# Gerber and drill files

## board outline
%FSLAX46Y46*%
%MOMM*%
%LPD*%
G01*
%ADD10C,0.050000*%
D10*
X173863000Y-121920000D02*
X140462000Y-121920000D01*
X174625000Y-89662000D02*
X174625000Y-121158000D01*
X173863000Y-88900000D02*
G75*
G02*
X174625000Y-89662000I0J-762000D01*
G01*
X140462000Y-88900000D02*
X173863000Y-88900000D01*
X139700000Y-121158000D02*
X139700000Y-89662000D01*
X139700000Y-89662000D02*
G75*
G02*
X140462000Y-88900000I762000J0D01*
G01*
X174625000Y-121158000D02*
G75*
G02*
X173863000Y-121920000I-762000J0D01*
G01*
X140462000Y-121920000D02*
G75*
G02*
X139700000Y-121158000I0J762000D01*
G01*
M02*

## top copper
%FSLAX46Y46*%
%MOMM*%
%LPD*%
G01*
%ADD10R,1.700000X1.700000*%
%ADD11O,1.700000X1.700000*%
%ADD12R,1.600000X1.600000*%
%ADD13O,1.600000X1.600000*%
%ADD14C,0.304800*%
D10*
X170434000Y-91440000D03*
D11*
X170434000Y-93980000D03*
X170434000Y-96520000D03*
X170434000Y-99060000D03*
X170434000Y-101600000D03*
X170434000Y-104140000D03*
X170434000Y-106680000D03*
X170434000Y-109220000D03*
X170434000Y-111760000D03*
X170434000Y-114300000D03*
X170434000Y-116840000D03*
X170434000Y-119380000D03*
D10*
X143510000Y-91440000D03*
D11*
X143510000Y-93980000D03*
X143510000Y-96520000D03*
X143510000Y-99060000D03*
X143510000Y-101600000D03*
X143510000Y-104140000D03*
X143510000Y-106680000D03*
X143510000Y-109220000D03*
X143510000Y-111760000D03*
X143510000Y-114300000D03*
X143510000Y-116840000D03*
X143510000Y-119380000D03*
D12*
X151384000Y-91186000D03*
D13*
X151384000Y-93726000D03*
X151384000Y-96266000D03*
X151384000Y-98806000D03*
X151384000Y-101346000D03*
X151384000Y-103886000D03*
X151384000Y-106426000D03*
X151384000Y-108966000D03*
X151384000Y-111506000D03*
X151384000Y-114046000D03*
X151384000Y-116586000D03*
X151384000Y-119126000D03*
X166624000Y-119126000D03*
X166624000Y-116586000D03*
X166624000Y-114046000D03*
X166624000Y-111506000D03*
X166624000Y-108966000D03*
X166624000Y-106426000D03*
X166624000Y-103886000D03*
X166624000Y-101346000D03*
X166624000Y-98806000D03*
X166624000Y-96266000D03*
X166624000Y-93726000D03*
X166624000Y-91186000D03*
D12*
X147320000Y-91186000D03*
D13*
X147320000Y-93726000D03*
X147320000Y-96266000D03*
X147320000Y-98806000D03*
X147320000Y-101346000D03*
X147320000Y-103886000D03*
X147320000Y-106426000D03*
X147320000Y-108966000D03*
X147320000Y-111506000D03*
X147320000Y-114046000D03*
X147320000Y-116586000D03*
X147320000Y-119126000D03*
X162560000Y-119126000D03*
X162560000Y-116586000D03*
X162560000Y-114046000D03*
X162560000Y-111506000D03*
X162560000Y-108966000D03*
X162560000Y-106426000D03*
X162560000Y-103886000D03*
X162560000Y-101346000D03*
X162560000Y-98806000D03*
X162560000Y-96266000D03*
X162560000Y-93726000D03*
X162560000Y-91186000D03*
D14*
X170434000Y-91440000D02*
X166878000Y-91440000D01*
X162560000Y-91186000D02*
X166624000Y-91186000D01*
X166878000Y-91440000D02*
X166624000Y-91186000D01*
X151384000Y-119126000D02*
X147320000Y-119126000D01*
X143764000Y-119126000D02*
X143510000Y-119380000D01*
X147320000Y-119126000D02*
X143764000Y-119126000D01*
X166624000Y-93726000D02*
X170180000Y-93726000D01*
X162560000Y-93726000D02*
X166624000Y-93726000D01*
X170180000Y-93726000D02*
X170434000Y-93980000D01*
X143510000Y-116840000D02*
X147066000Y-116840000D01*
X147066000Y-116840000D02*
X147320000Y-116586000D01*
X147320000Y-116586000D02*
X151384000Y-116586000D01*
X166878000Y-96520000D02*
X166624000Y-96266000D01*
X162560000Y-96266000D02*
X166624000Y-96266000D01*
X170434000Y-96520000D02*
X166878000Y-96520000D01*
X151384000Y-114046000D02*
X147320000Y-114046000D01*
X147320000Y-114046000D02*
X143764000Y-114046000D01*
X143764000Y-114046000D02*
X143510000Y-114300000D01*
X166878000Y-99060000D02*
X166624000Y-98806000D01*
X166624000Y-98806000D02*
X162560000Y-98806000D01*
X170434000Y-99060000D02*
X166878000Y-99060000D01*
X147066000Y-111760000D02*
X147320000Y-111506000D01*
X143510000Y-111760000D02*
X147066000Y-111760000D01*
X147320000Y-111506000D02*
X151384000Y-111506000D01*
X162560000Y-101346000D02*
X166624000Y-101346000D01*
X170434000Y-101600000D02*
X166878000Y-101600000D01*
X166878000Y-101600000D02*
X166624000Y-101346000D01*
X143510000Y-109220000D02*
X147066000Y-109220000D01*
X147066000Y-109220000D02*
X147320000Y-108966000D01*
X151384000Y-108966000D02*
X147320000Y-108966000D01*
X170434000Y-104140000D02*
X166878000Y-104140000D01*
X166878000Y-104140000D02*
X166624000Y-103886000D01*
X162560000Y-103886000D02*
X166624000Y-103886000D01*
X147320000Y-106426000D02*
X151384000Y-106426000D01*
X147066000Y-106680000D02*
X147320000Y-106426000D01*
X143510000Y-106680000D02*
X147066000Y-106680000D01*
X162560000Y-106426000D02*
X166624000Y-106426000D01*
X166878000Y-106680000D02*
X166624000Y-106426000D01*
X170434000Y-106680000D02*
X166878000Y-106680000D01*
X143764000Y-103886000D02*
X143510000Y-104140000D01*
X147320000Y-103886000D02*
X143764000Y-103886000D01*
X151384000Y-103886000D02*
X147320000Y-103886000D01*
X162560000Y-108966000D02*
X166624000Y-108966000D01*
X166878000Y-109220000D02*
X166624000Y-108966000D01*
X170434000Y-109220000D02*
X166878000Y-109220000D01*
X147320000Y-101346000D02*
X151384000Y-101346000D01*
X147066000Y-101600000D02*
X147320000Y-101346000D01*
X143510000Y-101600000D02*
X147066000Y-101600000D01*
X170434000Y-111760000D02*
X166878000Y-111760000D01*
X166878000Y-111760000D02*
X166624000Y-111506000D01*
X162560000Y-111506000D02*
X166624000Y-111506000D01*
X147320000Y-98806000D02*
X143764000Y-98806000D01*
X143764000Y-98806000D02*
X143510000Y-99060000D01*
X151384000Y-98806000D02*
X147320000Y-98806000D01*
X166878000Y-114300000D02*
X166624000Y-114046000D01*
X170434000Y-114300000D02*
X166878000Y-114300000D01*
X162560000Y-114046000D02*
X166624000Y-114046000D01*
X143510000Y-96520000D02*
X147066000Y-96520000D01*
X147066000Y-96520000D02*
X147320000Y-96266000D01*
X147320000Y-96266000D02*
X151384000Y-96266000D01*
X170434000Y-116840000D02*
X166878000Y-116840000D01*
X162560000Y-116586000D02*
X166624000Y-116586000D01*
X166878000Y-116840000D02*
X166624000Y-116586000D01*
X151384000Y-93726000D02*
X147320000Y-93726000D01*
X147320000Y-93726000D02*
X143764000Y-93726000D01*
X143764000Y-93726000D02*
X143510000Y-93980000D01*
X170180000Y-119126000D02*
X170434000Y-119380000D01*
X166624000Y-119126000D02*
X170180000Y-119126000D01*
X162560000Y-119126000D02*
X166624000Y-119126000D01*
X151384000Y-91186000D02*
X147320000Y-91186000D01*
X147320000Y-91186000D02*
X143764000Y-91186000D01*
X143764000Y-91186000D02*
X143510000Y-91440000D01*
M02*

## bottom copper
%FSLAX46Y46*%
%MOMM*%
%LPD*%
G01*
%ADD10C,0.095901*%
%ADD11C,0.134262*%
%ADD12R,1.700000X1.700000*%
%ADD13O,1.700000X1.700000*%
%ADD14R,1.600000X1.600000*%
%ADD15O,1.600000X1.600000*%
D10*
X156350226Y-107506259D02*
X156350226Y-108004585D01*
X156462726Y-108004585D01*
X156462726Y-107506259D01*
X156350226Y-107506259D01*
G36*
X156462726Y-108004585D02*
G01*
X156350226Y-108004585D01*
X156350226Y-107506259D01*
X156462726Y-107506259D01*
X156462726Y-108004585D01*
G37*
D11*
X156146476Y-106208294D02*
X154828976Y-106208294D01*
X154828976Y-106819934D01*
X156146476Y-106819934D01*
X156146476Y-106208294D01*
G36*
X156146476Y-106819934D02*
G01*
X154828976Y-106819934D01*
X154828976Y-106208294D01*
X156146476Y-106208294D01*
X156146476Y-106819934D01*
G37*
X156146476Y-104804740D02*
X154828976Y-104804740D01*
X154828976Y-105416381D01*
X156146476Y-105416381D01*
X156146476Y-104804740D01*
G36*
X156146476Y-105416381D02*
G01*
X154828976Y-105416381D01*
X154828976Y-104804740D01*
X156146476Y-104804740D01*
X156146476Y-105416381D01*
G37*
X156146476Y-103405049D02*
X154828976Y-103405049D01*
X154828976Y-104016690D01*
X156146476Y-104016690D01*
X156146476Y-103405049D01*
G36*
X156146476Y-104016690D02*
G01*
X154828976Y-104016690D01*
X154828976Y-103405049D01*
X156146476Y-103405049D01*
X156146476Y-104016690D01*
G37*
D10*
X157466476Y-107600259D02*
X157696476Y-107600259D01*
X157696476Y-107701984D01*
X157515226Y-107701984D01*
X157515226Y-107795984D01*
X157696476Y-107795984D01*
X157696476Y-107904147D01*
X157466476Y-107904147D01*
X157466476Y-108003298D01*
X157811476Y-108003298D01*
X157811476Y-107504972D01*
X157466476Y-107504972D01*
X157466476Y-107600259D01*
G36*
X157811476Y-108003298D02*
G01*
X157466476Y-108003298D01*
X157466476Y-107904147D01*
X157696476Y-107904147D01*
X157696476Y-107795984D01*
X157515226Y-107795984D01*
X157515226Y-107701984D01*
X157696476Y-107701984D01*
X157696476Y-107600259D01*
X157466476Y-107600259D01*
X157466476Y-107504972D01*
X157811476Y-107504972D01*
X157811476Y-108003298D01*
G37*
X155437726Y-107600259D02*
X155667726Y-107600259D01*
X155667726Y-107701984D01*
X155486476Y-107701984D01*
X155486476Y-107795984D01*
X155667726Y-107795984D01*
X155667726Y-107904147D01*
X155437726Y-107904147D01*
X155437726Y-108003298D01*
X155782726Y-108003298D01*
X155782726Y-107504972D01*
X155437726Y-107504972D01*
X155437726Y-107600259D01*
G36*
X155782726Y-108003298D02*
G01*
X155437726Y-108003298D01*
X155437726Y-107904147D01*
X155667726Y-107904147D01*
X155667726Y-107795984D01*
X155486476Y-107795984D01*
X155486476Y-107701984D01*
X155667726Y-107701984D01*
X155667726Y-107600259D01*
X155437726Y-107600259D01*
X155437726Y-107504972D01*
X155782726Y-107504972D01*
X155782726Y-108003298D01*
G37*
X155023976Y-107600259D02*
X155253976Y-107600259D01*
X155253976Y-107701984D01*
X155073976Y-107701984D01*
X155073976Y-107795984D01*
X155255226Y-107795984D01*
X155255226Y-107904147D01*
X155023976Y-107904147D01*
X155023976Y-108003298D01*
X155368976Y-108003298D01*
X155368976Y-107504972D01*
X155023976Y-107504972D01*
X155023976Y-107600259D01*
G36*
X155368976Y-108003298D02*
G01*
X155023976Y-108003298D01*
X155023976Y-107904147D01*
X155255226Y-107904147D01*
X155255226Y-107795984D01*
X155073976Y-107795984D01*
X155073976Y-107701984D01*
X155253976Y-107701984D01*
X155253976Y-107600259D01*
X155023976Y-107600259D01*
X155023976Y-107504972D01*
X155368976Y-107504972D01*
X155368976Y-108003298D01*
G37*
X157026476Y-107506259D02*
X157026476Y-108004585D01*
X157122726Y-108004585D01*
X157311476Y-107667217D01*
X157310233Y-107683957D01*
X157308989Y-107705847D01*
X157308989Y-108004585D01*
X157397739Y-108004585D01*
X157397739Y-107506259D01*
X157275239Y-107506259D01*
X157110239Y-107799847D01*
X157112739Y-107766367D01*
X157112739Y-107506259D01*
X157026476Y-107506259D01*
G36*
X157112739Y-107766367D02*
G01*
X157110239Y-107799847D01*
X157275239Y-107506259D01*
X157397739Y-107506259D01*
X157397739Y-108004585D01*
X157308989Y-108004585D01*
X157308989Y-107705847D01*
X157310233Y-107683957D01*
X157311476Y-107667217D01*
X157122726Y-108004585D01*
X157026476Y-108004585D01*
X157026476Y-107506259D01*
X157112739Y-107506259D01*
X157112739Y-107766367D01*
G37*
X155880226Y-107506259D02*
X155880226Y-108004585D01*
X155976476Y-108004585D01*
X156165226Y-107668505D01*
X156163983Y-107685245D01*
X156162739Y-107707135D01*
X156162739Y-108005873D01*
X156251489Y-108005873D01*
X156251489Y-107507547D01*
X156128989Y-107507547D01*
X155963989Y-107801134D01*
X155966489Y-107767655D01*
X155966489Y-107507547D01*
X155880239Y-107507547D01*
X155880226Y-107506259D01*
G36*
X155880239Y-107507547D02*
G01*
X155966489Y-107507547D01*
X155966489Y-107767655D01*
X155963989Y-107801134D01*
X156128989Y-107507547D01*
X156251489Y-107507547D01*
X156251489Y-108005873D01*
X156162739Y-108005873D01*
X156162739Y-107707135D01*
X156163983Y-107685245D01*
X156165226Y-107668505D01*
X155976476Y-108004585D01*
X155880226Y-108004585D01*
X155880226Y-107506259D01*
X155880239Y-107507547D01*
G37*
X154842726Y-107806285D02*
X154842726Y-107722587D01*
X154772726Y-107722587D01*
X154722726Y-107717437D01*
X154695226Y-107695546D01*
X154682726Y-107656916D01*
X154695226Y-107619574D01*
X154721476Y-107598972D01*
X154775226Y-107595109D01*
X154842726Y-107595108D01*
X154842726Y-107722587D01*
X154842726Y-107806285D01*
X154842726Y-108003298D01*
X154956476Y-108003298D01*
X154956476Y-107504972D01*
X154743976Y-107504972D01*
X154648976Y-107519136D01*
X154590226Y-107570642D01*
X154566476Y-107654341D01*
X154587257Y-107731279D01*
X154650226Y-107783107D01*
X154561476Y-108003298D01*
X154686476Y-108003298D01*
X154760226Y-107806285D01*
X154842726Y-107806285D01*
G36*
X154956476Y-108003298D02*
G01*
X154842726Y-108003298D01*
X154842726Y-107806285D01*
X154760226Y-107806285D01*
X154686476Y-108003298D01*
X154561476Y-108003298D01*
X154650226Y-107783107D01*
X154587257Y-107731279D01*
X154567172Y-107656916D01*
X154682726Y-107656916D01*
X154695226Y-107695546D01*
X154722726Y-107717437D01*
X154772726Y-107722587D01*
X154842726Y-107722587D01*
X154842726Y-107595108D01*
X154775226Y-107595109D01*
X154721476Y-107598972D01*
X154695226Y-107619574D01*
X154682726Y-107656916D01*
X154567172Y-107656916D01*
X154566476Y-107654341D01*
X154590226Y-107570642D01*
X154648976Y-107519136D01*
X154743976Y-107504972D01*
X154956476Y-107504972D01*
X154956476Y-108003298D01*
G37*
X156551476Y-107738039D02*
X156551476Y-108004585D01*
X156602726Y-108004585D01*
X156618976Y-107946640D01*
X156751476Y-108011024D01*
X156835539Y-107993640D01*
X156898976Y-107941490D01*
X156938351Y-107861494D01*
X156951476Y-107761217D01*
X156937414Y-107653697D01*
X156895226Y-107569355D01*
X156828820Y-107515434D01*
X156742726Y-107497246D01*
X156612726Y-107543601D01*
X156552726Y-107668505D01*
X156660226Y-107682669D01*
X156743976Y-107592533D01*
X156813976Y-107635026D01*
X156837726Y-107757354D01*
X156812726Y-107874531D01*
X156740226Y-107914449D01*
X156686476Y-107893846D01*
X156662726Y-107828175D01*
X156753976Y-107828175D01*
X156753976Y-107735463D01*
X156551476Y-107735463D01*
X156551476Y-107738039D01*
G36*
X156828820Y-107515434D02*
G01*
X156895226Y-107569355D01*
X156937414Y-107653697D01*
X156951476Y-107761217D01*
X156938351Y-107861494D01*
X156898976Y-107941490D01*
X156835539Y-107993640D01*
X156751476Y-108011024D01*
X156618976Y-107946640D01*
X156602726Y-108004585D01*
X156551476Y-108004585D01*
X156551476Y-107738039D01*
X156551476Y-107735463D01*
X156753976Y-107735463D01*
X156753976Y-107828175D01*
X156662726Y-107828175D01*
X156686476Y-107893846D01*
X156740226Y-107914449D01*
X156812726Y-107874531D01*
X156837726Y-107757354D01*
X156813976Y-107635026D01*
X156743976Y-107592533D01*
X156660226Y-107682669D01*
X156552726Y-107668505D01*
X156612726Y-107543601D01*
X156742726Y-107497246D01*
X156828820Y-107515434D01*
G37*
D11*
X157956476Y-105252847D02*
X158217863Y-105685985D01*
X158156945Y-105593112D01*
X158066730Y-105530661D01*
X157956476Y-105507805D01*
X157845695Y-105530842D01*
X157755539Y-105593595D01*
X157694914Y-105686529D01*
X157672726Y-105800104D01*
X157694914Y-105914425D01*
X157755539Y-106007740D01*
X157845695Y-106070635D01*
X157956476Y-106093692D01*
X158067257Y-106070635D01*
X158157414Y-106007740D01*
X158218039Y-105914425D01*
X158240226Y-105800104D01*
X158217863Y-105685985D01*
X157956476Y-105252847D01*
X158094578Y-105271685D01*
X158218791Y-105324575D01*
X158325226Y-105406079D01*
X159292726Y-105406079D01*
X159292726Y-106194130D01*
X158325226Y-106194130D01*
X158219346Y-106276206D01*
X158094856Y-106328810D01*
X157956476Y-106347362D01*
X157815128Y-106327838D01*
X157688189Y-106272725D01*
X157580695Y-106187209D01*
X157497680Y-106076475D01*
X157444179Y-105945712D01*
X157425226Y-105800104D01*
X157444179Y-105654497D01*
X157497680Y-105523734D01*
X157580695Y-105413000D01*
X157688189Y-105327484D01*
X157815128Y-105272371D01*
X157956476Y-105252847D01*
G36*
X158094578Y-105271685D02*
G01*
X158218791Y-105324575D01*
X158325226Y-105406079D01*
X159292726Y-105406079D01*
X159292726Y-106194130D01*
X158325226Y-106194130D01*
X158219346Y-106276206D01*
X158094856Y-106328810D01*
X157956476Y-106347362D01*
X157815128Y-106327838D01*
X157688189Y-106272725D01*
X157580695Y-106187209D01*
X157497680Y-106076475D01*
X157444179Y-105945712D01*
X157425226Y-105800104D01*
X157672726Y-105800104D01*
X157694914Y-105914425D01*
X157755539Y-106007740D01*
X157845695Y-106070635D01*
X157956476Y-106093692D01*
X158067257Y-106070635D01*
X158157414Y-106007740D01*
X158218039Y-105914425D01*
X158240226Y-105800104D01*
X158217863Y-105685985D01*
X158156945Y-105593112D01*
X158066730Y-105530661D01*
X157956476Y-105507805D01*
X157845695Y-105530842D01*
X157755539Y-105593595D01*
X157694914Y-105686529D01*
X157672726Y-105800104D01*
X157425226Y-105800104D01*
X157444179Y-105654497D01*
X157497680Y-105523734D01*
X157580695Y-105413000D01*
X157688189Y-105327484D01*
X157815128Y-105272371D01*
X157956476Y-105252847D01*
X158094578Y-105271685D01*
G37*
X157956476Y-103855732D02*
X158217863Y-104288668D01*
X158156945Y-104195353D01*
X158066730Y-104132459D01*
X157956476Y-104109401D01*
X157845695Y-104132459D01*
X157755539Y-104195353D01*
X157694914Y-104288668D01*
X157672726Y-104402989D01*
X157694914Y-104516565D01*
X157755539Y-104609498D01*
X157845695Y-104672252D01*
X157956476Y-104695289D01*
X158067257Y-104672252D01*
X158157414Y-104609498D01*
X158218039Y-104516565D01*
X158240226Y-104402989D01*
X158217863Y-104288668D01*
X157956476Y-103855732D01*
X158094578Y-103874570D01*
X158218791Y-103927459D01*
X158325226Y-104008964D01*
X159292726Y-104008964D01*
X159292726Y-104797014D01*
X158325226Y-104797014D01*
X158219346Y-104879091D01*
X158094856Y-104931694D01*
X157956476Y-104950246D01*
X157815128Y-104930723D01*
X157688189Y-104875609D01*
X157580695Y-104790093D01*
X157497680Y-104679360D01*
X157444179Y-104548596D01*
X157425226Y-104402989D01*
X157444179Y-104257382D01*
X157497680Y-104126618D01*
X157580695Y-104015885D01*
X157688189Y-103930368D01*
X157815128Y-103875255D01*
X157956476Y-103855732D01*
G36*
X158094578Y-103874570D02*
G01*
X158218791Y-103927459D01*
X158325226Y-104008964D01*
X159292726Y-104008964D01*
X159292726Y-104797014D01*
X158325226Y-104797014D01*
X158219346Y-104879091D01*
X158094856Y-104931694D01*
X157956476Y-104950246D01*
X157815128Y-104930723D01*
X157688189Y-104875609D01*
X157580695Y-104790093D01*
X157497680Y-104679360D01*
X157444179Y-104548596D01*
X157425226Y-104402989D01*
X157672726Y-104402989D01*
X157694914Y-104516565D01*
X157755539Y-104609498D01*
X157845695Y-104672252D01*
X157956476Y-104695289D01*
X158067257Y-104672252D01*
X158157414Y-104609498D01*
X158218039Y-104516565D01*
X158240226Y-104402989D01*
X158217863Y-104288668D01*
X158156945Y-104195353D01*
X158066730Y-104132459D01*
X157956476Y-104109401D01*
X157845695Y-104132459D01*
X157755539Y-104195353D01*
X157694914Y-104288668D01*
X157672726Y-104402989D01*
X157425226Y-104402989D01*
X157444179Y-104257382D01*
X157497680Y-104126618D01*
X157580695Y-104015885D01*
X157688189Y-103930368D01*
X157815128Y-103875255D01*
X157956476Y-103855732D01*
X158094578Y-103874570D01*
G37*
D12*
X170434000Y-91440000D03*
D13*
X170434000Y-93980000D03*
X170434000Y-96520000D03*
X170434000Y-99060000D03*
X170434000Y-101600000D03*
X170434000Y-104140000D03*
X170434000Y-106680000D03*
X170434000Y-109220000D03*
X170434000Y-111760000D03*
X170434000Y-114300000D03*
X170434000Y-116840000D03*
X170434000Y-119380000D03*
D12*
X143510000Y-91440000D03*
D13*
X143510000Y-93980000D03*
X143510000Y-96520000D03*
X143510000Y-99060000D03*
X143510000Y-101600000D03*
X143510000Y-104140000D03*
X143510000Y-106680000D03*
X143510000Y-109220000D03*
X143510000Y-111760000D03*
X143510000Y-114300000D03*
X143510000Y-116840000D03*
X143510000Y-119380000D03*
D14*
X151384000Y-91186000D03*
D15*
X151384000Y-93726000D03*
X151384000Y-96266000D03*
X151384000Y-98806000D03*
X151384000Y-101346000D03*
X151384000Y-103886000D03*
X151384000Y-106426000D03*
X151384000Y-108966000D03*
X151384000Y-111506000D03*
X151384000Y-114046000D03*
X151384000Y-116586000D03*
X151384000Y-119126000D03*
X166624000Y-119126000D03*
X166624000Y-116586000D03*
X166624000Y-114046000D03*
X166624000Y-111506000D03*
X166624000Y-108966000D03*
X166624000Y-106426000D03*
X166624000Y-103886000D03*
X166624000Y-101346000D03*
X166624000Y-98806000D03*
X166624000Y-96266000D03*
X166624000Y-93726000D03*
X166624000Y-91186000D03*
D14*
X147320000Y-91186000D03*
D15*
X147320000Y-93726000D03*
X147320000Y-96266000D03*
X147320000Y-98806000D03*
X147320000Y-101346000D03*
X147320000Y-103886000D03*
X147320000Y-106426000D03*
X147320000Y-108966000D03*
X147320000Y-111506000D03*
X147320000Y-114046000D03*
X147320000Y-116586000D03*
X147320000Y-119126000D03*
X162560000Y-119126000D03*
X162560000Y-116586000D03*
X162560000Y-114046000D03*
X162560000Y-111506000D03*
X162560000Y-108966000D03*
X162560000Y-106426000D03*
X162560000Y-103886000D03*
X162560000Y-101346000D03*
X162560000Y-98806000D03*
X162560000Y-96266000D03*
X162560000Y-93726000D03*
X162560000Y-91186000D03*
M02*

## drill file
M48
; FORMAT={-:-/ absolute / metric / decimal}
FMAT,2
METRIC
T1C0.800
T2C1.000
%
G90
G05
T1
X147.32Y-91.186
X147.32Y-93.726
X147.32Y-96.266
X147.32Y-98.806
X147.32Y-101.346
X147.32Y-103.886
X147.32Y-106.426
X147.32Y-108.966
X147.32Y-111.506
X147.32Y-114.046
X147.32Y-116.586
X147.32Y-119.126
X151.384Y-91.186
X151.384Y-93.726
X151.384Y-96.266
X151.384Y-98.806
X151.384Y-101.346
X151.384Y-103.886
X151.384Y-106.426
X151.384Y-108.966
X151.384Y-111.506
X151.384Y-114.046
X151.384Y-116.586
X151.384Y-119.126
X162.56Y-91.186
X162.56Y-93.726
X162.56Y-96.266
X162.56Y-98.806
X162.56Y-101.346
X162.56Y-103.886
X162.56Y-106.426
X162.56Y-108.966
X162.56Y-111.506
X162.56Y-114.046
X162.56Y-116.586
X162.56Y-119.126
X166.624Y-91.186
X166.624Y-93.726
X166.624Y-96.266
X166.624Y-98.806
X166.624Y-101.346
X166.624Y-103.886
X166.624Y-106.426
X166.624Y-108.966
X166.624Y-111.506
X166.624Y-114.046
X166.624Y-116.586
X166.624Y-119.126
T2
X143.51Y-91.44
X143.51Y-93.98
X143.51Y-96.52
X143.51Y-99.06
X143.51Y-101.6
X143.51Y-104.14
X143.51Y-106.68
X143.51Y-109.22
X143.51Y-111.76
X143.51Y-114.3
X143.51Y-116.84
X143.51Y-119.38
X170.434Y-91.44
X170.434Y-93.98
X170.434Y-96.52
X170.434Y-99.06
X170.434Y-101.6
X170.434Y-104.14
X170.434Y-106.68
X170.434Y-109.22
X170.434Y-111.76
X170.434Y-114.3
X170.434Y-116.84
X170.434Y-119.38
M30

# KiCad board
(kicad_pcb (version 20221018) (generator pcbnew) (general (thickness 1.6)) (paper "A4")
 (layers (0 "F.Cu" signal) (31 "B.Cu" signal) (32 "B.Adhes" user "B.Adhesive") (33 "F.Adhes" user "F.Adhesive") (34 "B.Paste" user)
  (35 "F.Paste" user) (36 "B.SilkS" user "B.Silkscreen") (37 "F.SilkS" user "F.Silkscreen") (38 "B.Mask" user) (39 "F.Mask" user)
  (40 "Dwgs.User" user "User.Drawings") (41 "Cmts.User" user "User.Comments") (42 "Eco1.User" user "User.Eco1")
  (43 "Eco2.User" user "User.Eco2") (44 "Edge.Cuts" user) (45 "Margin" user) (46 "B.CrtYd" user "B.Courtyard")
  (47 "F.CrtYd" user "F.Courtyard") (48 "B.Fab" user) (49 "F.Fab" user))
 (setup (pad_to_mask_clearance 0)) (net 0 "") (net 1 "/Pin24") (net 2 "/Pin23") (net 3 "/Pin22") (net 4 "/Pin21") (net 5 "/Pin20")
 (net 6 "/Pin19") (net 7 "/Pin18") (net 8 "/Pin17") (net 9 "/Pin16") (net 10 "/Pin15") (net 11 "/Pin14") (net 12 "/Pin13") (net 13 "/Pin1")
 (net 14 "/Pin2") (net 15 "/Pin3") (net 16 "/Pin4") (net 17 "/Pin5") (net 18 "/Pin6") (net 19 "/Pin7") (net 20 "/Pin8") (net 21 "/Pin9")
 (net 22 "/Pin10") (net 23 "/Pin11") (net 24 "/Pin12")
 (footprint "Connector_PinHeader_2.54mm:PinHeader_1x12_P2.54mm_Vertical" (layer "F.Cu") (at 170.434 91.44)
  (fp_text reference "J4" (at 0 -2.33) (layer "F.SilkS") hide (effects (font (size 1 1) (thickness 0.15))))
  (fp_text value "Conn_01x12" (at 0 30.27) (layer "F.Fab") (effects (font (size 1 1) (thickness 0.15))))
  (pad "1" thru_hole rect (at 0 0) (size 1.7 1.7) (drill 1) (layers "*.Cu" "*.Mask") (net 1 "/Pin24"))
  (pad "2" thru_hole oval (at 0 2.54) (size 1.7 1.7) (drill 1) (layers "*.Cu" "*.Mask") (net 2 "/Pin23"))
  (pad "3" thru_hole oval (at 0 5.08) (size 1.7 1.7) (drill 1) (layers "*.Cu" "*.Mask") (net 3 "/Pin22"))
  (pad "4" thru_hole oval (at 0 7.62) (size 1.7 1.7) (drill 1) (layers "*.Cu" "*.Mask") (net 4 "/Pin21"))
  (pad "5" thru_hole oval (at 0 10.16) (size 1.7 1.7) (drill 1) (layers "*.Cu" "*.Mask") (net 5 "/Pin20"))
  (pad "6" thru_hole oval (at 0 12.7) (size 1.7 1.7) (drill 1) (layers "*.Cu" "*.Mask") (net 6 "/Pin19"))
  (pad "7" thru_hole oval (at 0 15.24) (size 1.7 1.7) (drill 1) (layers "*.Cu" "*.Mask") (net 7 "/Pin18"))
  (pad "8" thru_hole oval (at 0 17.78) (size 1.7 1.7) (drill 1) (layers "*.Cu" "*.Mask") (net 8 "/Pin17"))
  (pad "9" thru_hole oval (at 0 20.32) (size 1.7 1.7) (drill 1) (layers "*.Cu" "*.Mask") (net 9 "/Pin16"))
  (pad "10" thru_hole oval (at 0 22.86) (size 1.7 1.7) (drill 1) (layers "*.Cu" "*.Mask") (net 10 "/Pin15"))
  (pad "11" thru_hole oval (at 0 25.4) (size 1.7 1.7) (drill 1) (layers "*.Cu" "*.Mask") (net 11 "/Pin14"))
  (pad "12" thru_hole oval (at 0 27.94) (size 1.7 1.7) (drill 1) (layers "*.Cu" "*.Mask") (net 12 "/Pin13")))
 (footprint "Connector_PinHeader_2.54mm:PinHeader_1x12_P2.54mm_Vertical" (layer "F.Cu") (at 143.51 91.44)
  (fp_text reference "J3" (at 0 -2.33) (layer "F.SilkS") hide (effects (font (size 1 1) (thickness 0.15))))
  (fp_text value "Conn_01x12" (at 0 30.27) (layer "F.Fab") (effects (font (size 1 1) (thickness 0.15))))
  (pad "1" thru_hole rect (at 0 0) (size 1.7 1.7) (drill 1) (layers "*.Cu" "*.Mask") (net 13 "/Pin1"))
  (pad "2" thru_hole oval (at 0 2.54) (size 1.7 1.7) (drill 1) (layers "*.Cu" "*.Mask") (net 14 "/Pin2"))
  (pad "3" thru_hole oval (at 0 5.08) (size 1.7 1.7) (drill 1) (layers "*.Cu" "*.Mask") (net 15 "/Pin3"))
  (pad "4" thru_hole oval (at 0 7.62) (size 1.7 1.7) (drill 1) (layers "*.Cu" "*.Mask") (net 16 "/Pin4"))
  (pad "5" thru_hole oval (at 0 10.16) (size 1.7 1.7) (drill 1) (layers "*.Cu" "*.Mask") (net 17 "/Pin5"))
  (pad "6" thru_hole oval (at 0 12.7) (size 1.7 1.7) (drill 1) (layers "*.Cu" "*.Mask") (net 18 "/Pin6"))
  (pad "7" thru_hole oval (at 0 15.24) (size 1.7 1.7) (drill 1) (layers "*.Cu" "*.Mask") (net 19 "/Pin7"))
  (pad "8" thru_hole oval (at 0 17.78) (size 1.7 1.7) (drill 1) (layers "*.Cu" "*.Mask") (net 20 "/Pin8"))
  (pad "9" thru_hole oval (at 0 20.32) (size 1.7 1.7) (drill 1) (layers "*.Cu" "*.Mask") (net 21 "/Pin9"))
  (pad "10" thru_hole oval (at 0 22.86) (size 1.7 1.7) (drill 1) (layers "*.Cu" "*.Mask") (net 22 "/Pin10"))
  (pad "11" thru_hole oval (at 0 25.4) (size 1.7 1.7) (drill 1) (layers "*.Cu" "*.Mask") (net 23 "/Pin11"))
  (pad "12" thru_hole oval (at 0 27.94) (size 1.7 1.7) (drill 1) (layers "*.Cu" "*.Mask") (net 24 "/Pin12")))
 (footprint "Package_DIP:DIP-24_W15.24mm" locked (layer "F.Cu") (at 151.384 91.186)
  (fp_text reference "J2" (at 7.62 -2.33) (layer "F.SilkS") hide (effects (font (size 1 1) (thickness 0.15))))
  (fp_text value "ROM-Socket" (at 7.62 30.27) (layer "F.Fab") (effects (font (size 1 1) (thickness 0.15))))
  (pad "1" thru_hole rect locked (at 0 0) (size 1.6 1.6) (drill 0.8) (layers "*.Cu" "*.Mask") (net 13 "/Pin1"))
  (pad "2" thru_hole oval locked (at 0 2.54) (size 1.6 1.6) (drill 0.8) (layers "*.Cu" "*.Mask") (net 14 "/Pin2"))
  (pad "3" thru_hole oval locked (at 0 5.08) (size 1.6 1.6) (drill 0.8) (layers "*.Cu" "*.Mask") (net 15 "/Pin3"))
  (pad "4" thru_hole oval locked (at 0 7.62) (size 1.6 1.6) (drill 0.8) (layers "*.Cu" "*.Mask") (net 16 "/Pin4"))
  (pad "5" thru_hole oval locked (at 0 10.16) (size 1.6 1.6) (drill 0.8) (layers "*.Cu" "*.Mask") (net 17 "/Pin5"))
  (pad "6" thru_hole oval locked (at 0 12.7) (size 1.6 1.6) (drill 0.8) (layers "*.Cu" "*.Mask") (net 18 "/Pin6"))
  (pad "7" thru_hole oval locked (at 0 15.24) (size 1.6 1.6) (drill 0.8) (layers "*.Cu" "*.Mask") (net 19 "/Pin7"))
  (pad "8" thru_hole oval locked (at 0 17.78) (size 1.6 1.6) (drill 0.8) (layers "*.Cu" "*.Mask") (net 20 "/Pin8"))
  (pad "9" thru_hole oval locked (at 0 20.32) (size 1.6 1.6) (drill 0.8) (layers "*.Cu" "*.Mask") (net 21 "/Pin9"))
  (pad "10" thru_hole oval locked (at 0 22.86) (size 1.6 1.6) (drill 0.8) (layers "*.Cu" "*.Mask") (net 22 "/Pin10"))
  (pad "11" thru_hole oval locked (at 0 25.4) (size 1.6 1.6) (drill 0.8) (layers "*.Cu" "*.Mask") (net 23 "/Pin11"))
  (pad "12" thru_hole oval locked (at 0 27.94) (size 1.6 1.6) (drill 0.8) (layers "*.Cu" "*.Mask") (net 24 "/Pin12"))
  (pad "13" thru_hole oval locked (at 15.24 27.94) (size 1.6 1.6) (drill 0.8) (layers "*.Cu" "*.Mask") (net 12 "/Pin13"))
  (pad "14" thru_hole oval locked (at 15.24 25.4) (size 1.6 1.6) (drill 0.8) (layers "*.Cu" "*.Mask") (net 11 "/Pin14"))
  (pad "15" thru_hole oval locked (at 15.24 22.86) (size 1.6 1.6) (drill 0.8) (layers "*.Cu" "*.Mask") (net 10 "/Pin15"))
  (pad "16" thru_hole oval locked (at 15.24 20.32) (size 1.6 1.6) (drill 0.8) (layers "*.Cu" "*.Mask") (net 9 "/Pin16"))
  (pad "17" thru_hole oval locked (at 15.24 17.78) (size 1.6 1.6) (drill 0.8) (layers "*.Cu" "*.Mask") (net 8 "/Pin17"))
  (pad "18" thru_hole oval locked (at 15.24 15.24) (size 1.6 1.6) (drill 0.8) (layers "*.Cu" "*.Mask") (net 7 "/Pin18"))
  (pad "19" thru_hole oval locked (at 15.24 12.7) (size 1.6 1.6) (drill 0.8) (layers "*.Cu" "*.Mask") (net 6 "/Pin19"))
  (pad "20" thru_hole oval locked (at 15.24 10.16) (size 1.6 1.6) (drill 0.8) (layers "*.Cu" "*.Mask") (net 5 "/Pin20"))
  (pad "21" thru_hole oval locked (at 15.24 7.62) (size 1.6 1.6) (drill 0.8) (layers "*.Cu" "*.Mask") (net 4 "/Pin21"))
  (pad "22" thru_hole oval locked (at 15.24 5.08) (size 1.6 1.6) (drill 0.8) (layers "*.Cu" "*.Mask") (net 3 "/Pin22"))
  (pad "23" thru_hole oval locked (at 15.24 2.54) (size 1.6 1.6) (drill 0.8) (layers "*.Cu" "*.Mask") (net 2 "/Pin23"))
  (pad "24" thru_hole oval locked (at 15.24 0) (size 1.6 1.6) (drill 0.8) (layers "*.Cu" "*.Mask") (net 1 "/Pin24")))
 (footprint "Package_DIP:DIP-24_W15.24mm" (layer "F.Cu") (at 147.32 91.186)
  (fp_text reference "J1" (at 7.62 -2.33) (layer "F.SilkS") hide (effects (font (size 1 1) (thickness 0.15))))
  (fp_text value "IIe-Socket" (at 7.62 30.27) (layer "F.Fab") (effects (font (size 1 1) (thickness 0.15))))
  (pad "1" thru_hole rect (at 0 0) (size 1.6 1.6) (drill 0.8) (layers "*.Cu" "*.Mask") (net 13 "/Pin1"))
  (pad "2" thru_hole oval (at 0 2.54) (size 1.6 1.6) (drill 0.8) (layers "*.Cu" "*.Mask") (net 14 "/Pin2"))
  (pad "3" thru_hole oval (at 0 5.08) (size 1.6 1.6) (drill 0.8) (layers "*.Cu" "*.Mask") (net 15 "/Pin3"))
  (pad "4" thru_hole oval (at 0 7.62) (size 1.6 1.6) (drill 0.8) (layers "*.Cu" "*.Mask") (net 16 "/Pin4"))
  (pad "5" thru_hole oval (at 0 10.16) (size 1.6 1.6) (drill 0.8) (layers "*.Cu" "*.Mask") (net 17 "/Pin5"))
  (pad "6" thru_hole oval (at 0 12.7) (size 1.6 1.6) (drill 0.8) (layers "*.Cu" "*.Mask") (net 18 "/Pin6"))
  (pad "7" thru_hole oval (at 0 15.24) (size 1.6 1.6) (drill 0.8) (layers "*.Cu" "*.Mask") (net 19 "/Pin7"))
  (pad "8" thru_hole oval (at 0 17.78) (size 1.6 1.6) (drill 0.8) (layers "*.Cu" "*.Mask") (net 20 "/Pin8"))
  (pad "9" thru_hole oval (at 0 20.32) (size 1.6 1.6) (drill 0.8) (layers "*.Cu" "*.Mask") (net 21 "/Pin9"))
  (pad "10" thru_hole oval (at 0 22.86) (size 1.6 1.6) (drill 0.8) (layers "*.Cu" "*.Mask") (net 22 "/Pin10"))
  (pad "11" thru_hole oval (at 0 25.4) (size 1.6 1.6) (drill 0.8) (layers "*.Cu" "*.Mask") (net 23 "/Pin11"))
  (pad "12" thru_hole oval (at 0 27.94) (size 1.6 1.6) (drill 0.8) (layers "*.Cu" "*.Mask") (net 24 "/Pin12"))
  (pad "13" thru_hole oval (at 15.24 27.94) (size 1.6 1.6) (drill 0.8) (layers "*.Cu" "*.Mask") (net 12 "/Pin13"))
  (pad "14" thru_hole oval (at 15.24 25.4) (size 1.6 1.6) (drill 0.8) (layers "*.Cu" "*.Mask") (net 11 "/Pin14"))
  (pad "15" thru_hole oval (at 15.24 22.86) (size 1.6 1.6) (drill 0.8) (layers "*.Cu" "*.Mask") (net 10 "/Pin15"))
  (pad "16" thru_hole oval (at 15.24 20.32) (size 1.6 1.6) (drill 0.8) (layers "*.Cu" "*.Mask") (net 9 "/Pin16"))
  (pad "17" thru_hole oval (at 15.24 17.78) (size 1.6 1.6) (drill 0.8) (layers "*.Cu" "*.Mask") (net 8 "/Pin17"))
  (pad "18" thru_hole oval (at 15.24 15.24) (size 1.6 1.6) (drill 0.8) (layers "*.Cu" "*.Mask") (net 7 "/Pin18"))
  (pad "19" thru_hole oval (at 15.24 12.7) (size 1.6 1.6) (drill 0.8) (layers "*.Cu" "*.Mask") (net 6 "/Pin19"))
  (pad "20" thru_hole oval (at 15.24 10.16) (size 1.6 1.6) (drill 0.8) (layers "*.Cu" "*.Mask") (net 5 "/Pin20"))
  (pad "21" thru_hole oval (at 15.24 7.62) (size 1.6 1.6) (drill 0.8) (layers "*.Cu" "*.Mask") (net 4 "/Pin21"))
  (pad "22" thru_hole oval (at 15.24 5.08) (size 1.6 1.6) (drill 0.8) (layers "*.Cu" "*.Mask") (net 3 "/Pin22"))
  (pad "23" thru_hole oval (at 15.24 2.54) (size 1.6 1.6) (drill 0.8) (layers "*.Cu" "*.Mask") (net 2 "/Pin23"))
  (pad "24" thru_hole oval (at 15.24 0) (size 1.6 1.6) (drill 0.8) (layers "*.Cu" "*.Mask") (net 1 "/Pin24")))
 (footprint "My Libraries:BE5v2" (layer "B.Cu") (at 159.561476 103.011024 180)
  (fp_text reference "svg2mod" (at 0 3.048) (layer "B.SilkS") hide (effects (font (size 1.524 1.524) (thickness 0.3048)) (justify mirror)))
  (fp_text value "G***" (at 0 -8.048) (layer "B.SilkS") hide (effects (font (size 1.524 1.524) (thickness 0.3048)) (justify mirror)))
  (fp_poly
   (pts (xy 3.21125 -4.495235) (xy 3.21125 -4.993561) (xy 3.09875 -4.993561) (xy 3.09875 -4.495235) (xy 3.21125 -4.495235))
   (stroke (width 0.095901) (type solid)) (fill solid) (layer "B.Cu"))
  (fp_poly
   (pts (xy 3.415 -3.19727) (xy 4.7325 -3.19727) (xy 4.7325 -3.80891) (xy 3.415 -3.80891) (xy 3.415 -3.19727))
   (stroke (width 0.134262) (type solid)) (fill solid) (layer "B.Cu"))
  (fp_poly
   (pts (xy 3.415 -1.793716) (xy 4.7325 -1.793716) (xy 4.7325 -2.405357) (xy 3.415 -2.405357) (xy 3.415 -1.793716))
   (stroke (width 0.134262) (type solid)) (fill solid) (layer "B.Cu"))
  (fp_poly
   (pts (xy 3.415 -0.394025) (xy 4.7325 -0.394025) (xy 4.7325 -1.005666) (xy 3.415 -1.005666) (xy 3.415 -0.394025))
   (stroke (width 0.134262) (type solid)) (fill solid) (layer "B.Cu"))
  (fp_poly
   (pts (xy 2.095 -4.589235) (xy 1.865 -4.589235) (xy 1.865 -4.69096) (xy 2.04625 -4.69096) (xy 2.04625 -4.78496) (xy 1.865 -4.78496)
    (xy 1.865 -4.893123) (xy 2.095 -4.893123) (xy 2.095 -4.992274) (xy 1.75 -4.992274) (xy 1.75 -4.493948) (xy 2.095 -4.493948)
    (xy 2.095 -4.589235))
   (stroke (width 0.095901) (type solid)) (fill solid) (layer "B.Cu"))
  (fp_poly
   (pts (xy 4.12375 -4.589235) (xy 3.89375 -4.589235) (xy 3.89375 -4.69096) (xy 4.075 -4.69096) (xy 4.075 -4.78496) (xy 3.89375 -4.78496)
    (xy 3.89375 -4.893123) (xy 4.12375 -4.893123) (xy 4.12375 -4.992274) (xy 3.77875 -4.992274) (xy 3.77875 -4.493948)
    (xy 4.12375 -4.493948) (xy 4.12375 -4.589235))
   (stroke (width 0.095901) (type solid)) (fill solid) (layer "B.Cu"))
  (fp_poly
   (pts (xy 4.5375 -4.589235) (xy 4.3075 -4.589235) (xy 4.3075 -4.69096) (xy 4.4875 -4.69096) (xy 4.4875 -4.78496) (xy 4.30625 -4.78496)
    (xy 4.30625 -4.893123) (xy 4.5375 -4.893123) (xy 4.5375 -4.992274) (xy 4.1925 -4.992274) (xy 4.1925 -4.493948) (xy 4.5375 -4.493948)
    (xy 4.5375 -4.589235))
   (stroke (width 0.095901) (type solid)) (fill solid) (layer "B.Cu"))
  (fp_poly
   (pts (xy 2.535 -4.495235) (xy 2.535 -4.993561) (xy 2.43875 -4.993561) (xy 2.25 -4.656193) (xy 2.251243 -4.672933) (xy 2.252487 -4.694823)
    (xy 2.252487 -4.993561) (xy 2.163737 -4.993561) (xy 2.163737 -4.495235) (xy 2.286237 -4.495235) (xy 2.451237 -4.788823)
    (xy 2.448737 -4.755343) (xy 2.448737 -4.495235) (xy 2.535 -4.495235))
   (stroke (width 0.095901) (type solid)) (fill solid) (layer "B.Cu"))
  (fp_poly
   (pts (xy 3.68125 -4.495235) (xy 3.68125 -4.993561) (xy 3.585 -4.993561) (xy 3.39625 -4.657481) (xy 3.397493 -4.674221)
    (xy 3.398737 -4.696111) (xy 3.398737 -4.994849) (xy 3.309987 -4.994849) (xy 3.309987 -4.496523) (xy 3.432487 -4.496523)
    (xy 3.597487 -4.79011) (xy 3.594987 -4.756631) (xy 3.594987 -4.496523) (xy 3.681237 -4.496523) (xy 3.68125 -4.495235))
   (stroke (width 0.095901) (type solid)) (fill solid) (layer "B.Cu"))
  (fp_poly
   (pts (xy 4.71875 -4.795261) (xy 4.71875 -4.711563) (xy 4.78875 -4.711563) (xy 4.83875 -4.706413) (xy 4.86625 -4.684522)
    (xy 4.87875 -4.645892) (xy 4.86625 -4.60855) (xy 4.84 -4.587948) (xy 4.78625 -4.584085) (xy 4.71875 -4.584084) (xy 4.71875 -4.711563)
    (xy 4.71875 -4.795261) (xy 4.71875 -4.992274) (xy 4.605 -4.992274) (xy 4.605 -4.493948) (xy 4.8175 -4.493948) (xy 4.9125 -4.508112)
    (xy 4.97125 -4.559618) (xy 4.995 -4.643317) (xy 4.974219 -4.720255) (xy 4.91125 -4.772083) (xy 5 -4.992274) (xy 4.875 -4.992274)
    (xy 4.80125 -4.795261) (xy 4.71875 -4.795261))
   (stroke (width 0.095901) (type solid)) (fill solid) (layer "B.Cu"))
  (fp_poly
   (pts (xy 3.01 -4.727015) (xy 3.01 -4.993561) (xy 2.95875 -4.993561) (xy 2.9425 -4.935616) (xy 2.81 -5) (xy 2.725937 -4.982616)
    (xy 2.6625 -4.930466) (xy 2.623125 -4.85047) (xy 2.61 -4.750193) (xy 2.624062 -4.642673) (xy 2.66625 -4.558331) (xy 2.732656 -4.50441)
    (xy 2.81875 -4.486222) (xy 2.94875 -4.532577) (xy 3.00875 -4.657481) (xy 2.90125 -4.671645) (xy 2.8175 -4.581509) (xy 2.7475 -4.624002)
    (xy 2.72375 -4.74633) (xy 2.74875 -4.863507) (xy 2.82125 -4.903425) (xy 2.875 -4.882822) (xy 2.89875 -4.817151) (xy 2.8075 -4.817151)
    (xy 2.8075 -4.724439) (xy 3.01 -4.724439) (xy 3.01 -4.727015))
   (stroke (width 0.095901) (type solid)) (fill solid) (layer "B.Cu"))
  (fp_poly
   (pts (xy 1.605 -2.241823) (xy 1.343613 -2.674961) (xy 1.404531 -2.582088) (xy 1.494746 -2.519637) (xy 1.605 -2.496781)
    (xy 1.715781 -2.519818) (xy 1.805937 -2.582571) (xy 1.866562 -2.675505) (xy 1.88875 -2.78908) (xy 1.866562 -2.903401)
    (xy 1.805937 -2.996716) (xy 1.715781 -3.059611) (xy 1.605 -3.082668) (xy 1.494219 -3.059611) (xy 1.404062 -2.996716)
    (xy 1.343437 -2.903401) (xy 1.32125 -2.78908) (xy 1.343613 -2.674961) (xy 1.605 -2.241823) (xy 1.466898 -2.260661)
    (xy 1.342685 -2.313551) (xy 1.23625 -2.395055) (xy 0.26875 -2.395055) (xy 0.26875 -3.183106) (xy 1.23625 -3.183106)
    (xy 1.34213 -3.265182) (xy 1.46662 -3.317786) (xy 1.605 -3.336338) (xy 1.746348 -3.316814) (xy 1.873287 -3.261701)
    (xy 1.980781 -3.176185) (xy 2.063796 -3.065451) (xy 2.117297 -2.934688) (xy 2.13625 -2.78908) (xy 2.117297 -2.643473)
    (xy 2.063796 -2.51271) (xy 1.980781 -2.401976) (xy 1.873287 -2.31646) (xy 1.746348 -2.261347) (xy 1.605 -2.241823))
   (stroke (width 0.134262) (type solid)) (fill solid) (layer "B.Cu"))
  (fp_poly
   (pts (xy 1.605 -0.844708) (xy 1.343613 -1.277644) (xy 1.404531 -1.184329) (xy 1.494746 -1.121435) (xy 1.605 -1.098377)
    (xy 1.715781 -1.121435) (xy 1.805937 -1.184329) (xy 1.866562 -1.277644) (xy 1.88875 -1.391965) (xy 1.866562 -1.505541)
    (xy 1.805937 -1.598474) (xy 1.715781 -1.661228) (xy 1.605 -1.684265) (xy 1.494219 -1.661228) (xy 1.404062 -1.598474)
    (xy 1.343437 -1.505541) (xy 1.32125 -1.391965) (xy 1.343613 -1.277644) (xy 1.605 -0.844708) (xy 1.466898 -0.863546)
    (xy 1.342685 -0.916435) (xy 1.23625 -0.99794) (xy 0.26875 -0.99794) (xy 0.26875 -1.78599) (xy 1.23625 -1.78599) (xy 1.34213 -1.868067)
    (xy 1.46662 -1.92067) (xy 1.605 -1.939222) (xy 1.746348 -1.919699) (xy 1.873287 -1.864585) (xy 1.980781 -1.779069)
    (xy 2.063796 -1.668336) (xy 2.117297 -1.537572) (xy 2.13625 -1.391965) (xy 2.117297 -1.246358) (xy 2.063796 -1.115594)
    (xy 1.980781 -1.004861) (xy 1.873287 -0.919344) (xy 1.746348 -0.864231) (xy 1.605 -0.844708))
   (stroke (width 0.134262) (type solid)) (fill solid) (layer "B.Cu")))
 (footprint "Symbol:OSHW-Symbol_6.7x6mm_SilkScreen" (layer "B.Cu") (at 157.0736 95.6818 180)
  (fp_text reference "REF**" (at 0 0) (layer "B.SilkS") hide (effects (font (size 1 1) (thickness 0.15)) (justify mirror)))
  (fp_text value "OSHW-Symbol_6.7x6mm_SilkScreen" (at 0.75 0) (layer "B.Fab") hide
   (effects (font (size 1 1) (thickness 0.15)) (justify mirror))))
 (gr_line (start 173.863 121.92) (end 140.462 121.92) (stroke (width 0.05) (type solid)) (layer "Edge.Cuts"))
 (gr_line (start 174.625 89.662) (end 174.625 121.158) (stroke (width 0.05) (type solid)) (layer "Edge.Cuts"))
 (gr_arc (start 173.863 88.9) (mid 174.401815 89.123185) (end 174.625 89.662) (stroke (width 0.05) (type solid)) (layer "Edge.Cuts"))
 (gr_line (start 140.462 88.9) (end 173.863 88.9) (stroke (width 0.05) (type solid)) (layer "Edge.Cuts"))
 (gr_line (start 139.7 121.158) (end 139.7 89.662) (stroke (width 0.05) (type solid)) (layer "Edge.Cuts"))
 (gr_arc (start 139.7 89.662) (mid 139.923185 89.123185) (end 140.462 88.9) (stroke (width 0.05) (type solid)) (layer "Edge.Cuts"))
 (gr_arc (start 174.625 121.158) (mid 174.401815 121.696815) (end 173.863 121.92) (stroke (width 0.05) (type solid)) (layer "Edge.Cuts"))
 (gr_arc (start 140.462 121.92) (mid 139.923185 121.696815) (end 139.7 121.158) (stroke (width 0.05) (type solid)) (layer "Edge.Cuts"))
 (segment (start 170.434 91.44) (end 166.878 91.44) (width 0.3048) (layer "F.Cu") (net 1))
 (segment (start 162.56 91.186) (end 166.624 91.186) (width 0.3048) (layer "F.Cu") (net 1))
 (segment (start 166.878 91.44) (end 166.624 91.186) (width 0.3048) (layer "F.Cu") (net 1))
 (segment (start 151.384 119.126) (end 147.32 119.126) (width 0.3048) (layer "F.Cu") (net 24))
 (segment (start 143.764 119.126) (end 143.51 119.38) (width 0.3048) (layer "F.Cu") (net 24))
 (segment (start 147.32 119.126) (end 143.764 119.126) (width 0.3048) (layer "F.Cu") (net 24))
 (segment (start 166.624 93.726) (end 170.18 93.726) (width 0.3048) (layer "F.Cu") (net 2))
 (segment (start 162.56 93.726) (end 166.624 93.726) (width 0.3048) (layer "F.Cu") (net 2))
 (segment (start 170.18 93.726) (end 170.434 93.98) (width 0.3048) (layer "F.Cu") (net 2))
 (segment (start 143.51 116.84) (end 147.066 116.84) (width 0.3048) (layer "F.Cu") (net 23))
 (segment (start 147.066 116.84) (end 147.32 116.586) (width 0.3048) (layer "F.Cu") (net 23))
 (segment (start 147.32 116.586) (end 151.384 116.586) (width 0.3048) (layer "F.Cu") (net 23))
 (segment (start 166.878 96.52) (end 166.624 96.266) (width 0.3048) (layer "F.Cu") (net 3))
 (segment (start 162.56 96.266) (end 166.624 96.266) (width 0.3048) (layer "F.Cu") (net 3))
 (segment (start 170.434 96.52) (end 166.878 96.52) (width 0.3048) (layer "F.Cu") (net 3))
 (segment (start 151.384 114.046) (end 147.32 114.046) (width 0.3048) (layer "F.Cu") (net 22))
 (segment (start 147.32 114.046) (end 143.764 114.046) (width 0.3048) (layer "F.Cu") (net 22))
 (segment (start 143.764 114.046) (end 143.51 114.3) (width 0.3048) (layer "F.Cu") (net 22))
 (segment (start 166.878 99.06) (end 166.624 98.806) (width 0.3048) (layer "F.Cu") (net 4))
 (segment (start 166.624 98.806) (end 162.56 98.806) (width 0.3048) (layer "F.Cu") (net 4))
 (segment (start 170.434 99.06) (end 166.878 99.06) (width 0.3048) (layer "F.Cu") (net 4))
 (segment (start 147.066 111.76) (end 147.32 111.506) (width 0.3048) (layer "F.Cu") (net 21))
 (segment (start 143.51 111.76) (end 147.066 111.76) (width 0.3048) (layer "F.Cu") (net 21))
 (segment (start 147.32 111.506) (end 151.384 111.506) (width 0.3048) (layer "F.Cu") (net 21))
 (segment (start 162.56 101.346) (end 166.624 101.346) (width 0.3048) (layer "F.Cu") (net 5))
 (segment (start 170.434 101.6) (end 166.878 101.6) (width 0.3048) (layer "F.Cu") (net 5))
 (segment (start 166.878 101.6) (end 166.624 101.346) (width 0.3048) (layer "F.Cu") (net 5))
 (segment (start 143.51 109.22) (end 147.066 109.22) (width 0.3048) (layer "F.Cu") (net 20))
 (segment (start 147.066 109.22) (end 147.32 108.966) (width 0.3048) (layer "F.Cu") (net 20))
 (segment (start 151.384 108.966) (end 147.32 108.966) (width 0.3048) (layer "F.Cu") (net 20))
 (segment (start 170.434 104.14) (end 166.878 104.14) (width 0.3048) (layer "F.Cu") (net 6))
 (segment (start 166.878 104.14) (end 166.624 103.886) (width 0.3048) (layer "F.Cu") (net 6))
 (segment (start 162.56 103.886) (end 166.624 103.886) (width 0.3048) (layer "F.Cu") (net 6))
 (segment (start 147.32 106.426) (end 151.384 106.426) (width 0.3048) (layer "F.Cu") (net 19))
 (segment (start 147.066 106.68) (end 147.32 106.426) (width 0.3048) (layer "F.Cu") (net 19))
 (segment (start 143.51 106.68) (end 147.066 106.68) (width 0.3048) (layer "F.Cu") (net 19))
 (segment (start 162.56 106.426) (end 166.624 106.426) (width 0.3048) (layer "F.Cu") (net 7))
 (segment (start 166.878 106.68) (end 166.624 106.426) (width 0.3048) (layer "F.Cu") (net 7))
 (segment (start 170.434 106.68) (end 166.878 106.68) (width 0.3048) (layer "F.Cu") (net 7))
 (segment (start 143.764 103.886) (end 143.51 104.14) (width 0.3048) (layer "F.Cu") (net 18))
 (segment (start 147.32 103.886) (end 143.764 103.886) (width 0.3048) (layer "F.Cu") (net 18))
 (segment (start 151.384 103.886) (end 147.32 103.886) (width 0.3048) (layer "F.Cu") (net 18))
 (segment (start 162.56 108.966) (end 166.624 108.966) (width 0.3048) (layer "F.Cu") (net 8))
 (segment (start 166.878 109.22) (end 166.624 108.966) (width 0.3048) (layer "F.Cu") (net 8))
 (segment (start 170.434 109.22) (end 166.878 109.22) (width 0.3048) (layer "F.Cu") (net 8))
 (segment (start 147.32 101.346) (end 151.384 101.346) (width 0.3048) (layer "F.Cu") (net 17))
 (segment (start 147.066 101.6) (end 147.32 101.346) (width 0.3048) (layer "F.Cu") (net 17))
 (segment (start 143.51 101.6) (end 147.066 101.6) (width 0.3048) (layer "F.Cu") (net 17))
 (segment (start 170.434 111.76) (end 166.878 111.76) (width 0.3048) (layer "F.Cu") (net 9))
 (segment (start 166.878 111.76) (end 166.624 111.506) (width 0.3048) (layer "F.Cu") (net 9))
 (segment (start 162.56 111.506) (end 166.624 111.506) (width 0.3048) (layer "F.Cu") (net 9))
 (segment (start 147.32 98.806) (end 143.764 98.806) (width 0.3048) (layer "F.Cu") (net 16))
 (segment (start 143.764 98.806) (end 143.51 99.06) (width 0.3048) (layer "F.Cu") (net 16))
 (segment (start 151.384 98.806) (end 147.32 98.806) (width 0.3048) (layer "F.Cu") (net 16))
 (segment (start 166.878 114.3) (end 166.624 114.046) (width 0.3048) (layer "F.Cu") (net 10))
 (segment (start 170.434 114.3) (end 166.878 114.3) (width 0.3048) (layer "F.Cu") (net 10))
 (segment (start 162.56 114.046) (end 166.624 114.046) (width 0.3048) (layer "F.Cu") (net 10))
 (segment (start 143.51 96.52) (end 147.066 96.52) (width 0.3048) (layer "F.Cu") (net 15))
 (segment (start 147.066 96.52) (end 147.32 96.266) (width 0.3048) (layer "F.Cu") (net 15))
 (segment (start 147.32 96.266) (end 151.384 96.266) (width 0.3048) (layer "F.Cu") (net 15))
 (segment (start 170.434 116.84) (end 166.878 116.84) (width 0.3048) (layer "F.Cu") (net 11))
 (segment (start 162.56 116.586) (end 166.624 116.586) (width 0.3048) (layer "F.Cu") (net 11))
 (segment (start 166.878 116.84) (end 166.624 116.586) (width 0.3048) (layer "F.Cu") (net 11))
 (segment (start 151.384 93.726) (end 147.32 93.726) (width 0.3048) (layer "F.Cu") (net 14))
 (segment (start 147.32 93.726) (end 143.764 93.726) (width 0.3048) (layer "F.Cu") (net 14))
 (segment (start 143.764 93.726) (end 143.51 93.98) (width 0.3048) (layer "F.Cu") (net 14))
 (segment (start 170.18 119.126) (end 170.434 119.38) (width 0.3048) (layer "F.Cu") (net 12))
 (segment (start 166.624 119.126) (end 170.18 119.126) (width 0.3048) (layer "F.Cu") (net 12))
 (segment (start 162.56 119.126) (end 166.624 119.126) (width 0.3048) (layer "F.Cu") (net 12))
 (segment (start 151.384 91.186) (end 147.32 91.186) (width 0.3048) (layer "F.Cu") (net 13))
 (segment (start 147.32 91.186) (end 143.764 91.186) (width 0.3048) (layer "F.Cu") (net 13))
 (segment (start 143.764 91.186) (end 143.51 91.44) (width 0.3048) (layer "F.Cu") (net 13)))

